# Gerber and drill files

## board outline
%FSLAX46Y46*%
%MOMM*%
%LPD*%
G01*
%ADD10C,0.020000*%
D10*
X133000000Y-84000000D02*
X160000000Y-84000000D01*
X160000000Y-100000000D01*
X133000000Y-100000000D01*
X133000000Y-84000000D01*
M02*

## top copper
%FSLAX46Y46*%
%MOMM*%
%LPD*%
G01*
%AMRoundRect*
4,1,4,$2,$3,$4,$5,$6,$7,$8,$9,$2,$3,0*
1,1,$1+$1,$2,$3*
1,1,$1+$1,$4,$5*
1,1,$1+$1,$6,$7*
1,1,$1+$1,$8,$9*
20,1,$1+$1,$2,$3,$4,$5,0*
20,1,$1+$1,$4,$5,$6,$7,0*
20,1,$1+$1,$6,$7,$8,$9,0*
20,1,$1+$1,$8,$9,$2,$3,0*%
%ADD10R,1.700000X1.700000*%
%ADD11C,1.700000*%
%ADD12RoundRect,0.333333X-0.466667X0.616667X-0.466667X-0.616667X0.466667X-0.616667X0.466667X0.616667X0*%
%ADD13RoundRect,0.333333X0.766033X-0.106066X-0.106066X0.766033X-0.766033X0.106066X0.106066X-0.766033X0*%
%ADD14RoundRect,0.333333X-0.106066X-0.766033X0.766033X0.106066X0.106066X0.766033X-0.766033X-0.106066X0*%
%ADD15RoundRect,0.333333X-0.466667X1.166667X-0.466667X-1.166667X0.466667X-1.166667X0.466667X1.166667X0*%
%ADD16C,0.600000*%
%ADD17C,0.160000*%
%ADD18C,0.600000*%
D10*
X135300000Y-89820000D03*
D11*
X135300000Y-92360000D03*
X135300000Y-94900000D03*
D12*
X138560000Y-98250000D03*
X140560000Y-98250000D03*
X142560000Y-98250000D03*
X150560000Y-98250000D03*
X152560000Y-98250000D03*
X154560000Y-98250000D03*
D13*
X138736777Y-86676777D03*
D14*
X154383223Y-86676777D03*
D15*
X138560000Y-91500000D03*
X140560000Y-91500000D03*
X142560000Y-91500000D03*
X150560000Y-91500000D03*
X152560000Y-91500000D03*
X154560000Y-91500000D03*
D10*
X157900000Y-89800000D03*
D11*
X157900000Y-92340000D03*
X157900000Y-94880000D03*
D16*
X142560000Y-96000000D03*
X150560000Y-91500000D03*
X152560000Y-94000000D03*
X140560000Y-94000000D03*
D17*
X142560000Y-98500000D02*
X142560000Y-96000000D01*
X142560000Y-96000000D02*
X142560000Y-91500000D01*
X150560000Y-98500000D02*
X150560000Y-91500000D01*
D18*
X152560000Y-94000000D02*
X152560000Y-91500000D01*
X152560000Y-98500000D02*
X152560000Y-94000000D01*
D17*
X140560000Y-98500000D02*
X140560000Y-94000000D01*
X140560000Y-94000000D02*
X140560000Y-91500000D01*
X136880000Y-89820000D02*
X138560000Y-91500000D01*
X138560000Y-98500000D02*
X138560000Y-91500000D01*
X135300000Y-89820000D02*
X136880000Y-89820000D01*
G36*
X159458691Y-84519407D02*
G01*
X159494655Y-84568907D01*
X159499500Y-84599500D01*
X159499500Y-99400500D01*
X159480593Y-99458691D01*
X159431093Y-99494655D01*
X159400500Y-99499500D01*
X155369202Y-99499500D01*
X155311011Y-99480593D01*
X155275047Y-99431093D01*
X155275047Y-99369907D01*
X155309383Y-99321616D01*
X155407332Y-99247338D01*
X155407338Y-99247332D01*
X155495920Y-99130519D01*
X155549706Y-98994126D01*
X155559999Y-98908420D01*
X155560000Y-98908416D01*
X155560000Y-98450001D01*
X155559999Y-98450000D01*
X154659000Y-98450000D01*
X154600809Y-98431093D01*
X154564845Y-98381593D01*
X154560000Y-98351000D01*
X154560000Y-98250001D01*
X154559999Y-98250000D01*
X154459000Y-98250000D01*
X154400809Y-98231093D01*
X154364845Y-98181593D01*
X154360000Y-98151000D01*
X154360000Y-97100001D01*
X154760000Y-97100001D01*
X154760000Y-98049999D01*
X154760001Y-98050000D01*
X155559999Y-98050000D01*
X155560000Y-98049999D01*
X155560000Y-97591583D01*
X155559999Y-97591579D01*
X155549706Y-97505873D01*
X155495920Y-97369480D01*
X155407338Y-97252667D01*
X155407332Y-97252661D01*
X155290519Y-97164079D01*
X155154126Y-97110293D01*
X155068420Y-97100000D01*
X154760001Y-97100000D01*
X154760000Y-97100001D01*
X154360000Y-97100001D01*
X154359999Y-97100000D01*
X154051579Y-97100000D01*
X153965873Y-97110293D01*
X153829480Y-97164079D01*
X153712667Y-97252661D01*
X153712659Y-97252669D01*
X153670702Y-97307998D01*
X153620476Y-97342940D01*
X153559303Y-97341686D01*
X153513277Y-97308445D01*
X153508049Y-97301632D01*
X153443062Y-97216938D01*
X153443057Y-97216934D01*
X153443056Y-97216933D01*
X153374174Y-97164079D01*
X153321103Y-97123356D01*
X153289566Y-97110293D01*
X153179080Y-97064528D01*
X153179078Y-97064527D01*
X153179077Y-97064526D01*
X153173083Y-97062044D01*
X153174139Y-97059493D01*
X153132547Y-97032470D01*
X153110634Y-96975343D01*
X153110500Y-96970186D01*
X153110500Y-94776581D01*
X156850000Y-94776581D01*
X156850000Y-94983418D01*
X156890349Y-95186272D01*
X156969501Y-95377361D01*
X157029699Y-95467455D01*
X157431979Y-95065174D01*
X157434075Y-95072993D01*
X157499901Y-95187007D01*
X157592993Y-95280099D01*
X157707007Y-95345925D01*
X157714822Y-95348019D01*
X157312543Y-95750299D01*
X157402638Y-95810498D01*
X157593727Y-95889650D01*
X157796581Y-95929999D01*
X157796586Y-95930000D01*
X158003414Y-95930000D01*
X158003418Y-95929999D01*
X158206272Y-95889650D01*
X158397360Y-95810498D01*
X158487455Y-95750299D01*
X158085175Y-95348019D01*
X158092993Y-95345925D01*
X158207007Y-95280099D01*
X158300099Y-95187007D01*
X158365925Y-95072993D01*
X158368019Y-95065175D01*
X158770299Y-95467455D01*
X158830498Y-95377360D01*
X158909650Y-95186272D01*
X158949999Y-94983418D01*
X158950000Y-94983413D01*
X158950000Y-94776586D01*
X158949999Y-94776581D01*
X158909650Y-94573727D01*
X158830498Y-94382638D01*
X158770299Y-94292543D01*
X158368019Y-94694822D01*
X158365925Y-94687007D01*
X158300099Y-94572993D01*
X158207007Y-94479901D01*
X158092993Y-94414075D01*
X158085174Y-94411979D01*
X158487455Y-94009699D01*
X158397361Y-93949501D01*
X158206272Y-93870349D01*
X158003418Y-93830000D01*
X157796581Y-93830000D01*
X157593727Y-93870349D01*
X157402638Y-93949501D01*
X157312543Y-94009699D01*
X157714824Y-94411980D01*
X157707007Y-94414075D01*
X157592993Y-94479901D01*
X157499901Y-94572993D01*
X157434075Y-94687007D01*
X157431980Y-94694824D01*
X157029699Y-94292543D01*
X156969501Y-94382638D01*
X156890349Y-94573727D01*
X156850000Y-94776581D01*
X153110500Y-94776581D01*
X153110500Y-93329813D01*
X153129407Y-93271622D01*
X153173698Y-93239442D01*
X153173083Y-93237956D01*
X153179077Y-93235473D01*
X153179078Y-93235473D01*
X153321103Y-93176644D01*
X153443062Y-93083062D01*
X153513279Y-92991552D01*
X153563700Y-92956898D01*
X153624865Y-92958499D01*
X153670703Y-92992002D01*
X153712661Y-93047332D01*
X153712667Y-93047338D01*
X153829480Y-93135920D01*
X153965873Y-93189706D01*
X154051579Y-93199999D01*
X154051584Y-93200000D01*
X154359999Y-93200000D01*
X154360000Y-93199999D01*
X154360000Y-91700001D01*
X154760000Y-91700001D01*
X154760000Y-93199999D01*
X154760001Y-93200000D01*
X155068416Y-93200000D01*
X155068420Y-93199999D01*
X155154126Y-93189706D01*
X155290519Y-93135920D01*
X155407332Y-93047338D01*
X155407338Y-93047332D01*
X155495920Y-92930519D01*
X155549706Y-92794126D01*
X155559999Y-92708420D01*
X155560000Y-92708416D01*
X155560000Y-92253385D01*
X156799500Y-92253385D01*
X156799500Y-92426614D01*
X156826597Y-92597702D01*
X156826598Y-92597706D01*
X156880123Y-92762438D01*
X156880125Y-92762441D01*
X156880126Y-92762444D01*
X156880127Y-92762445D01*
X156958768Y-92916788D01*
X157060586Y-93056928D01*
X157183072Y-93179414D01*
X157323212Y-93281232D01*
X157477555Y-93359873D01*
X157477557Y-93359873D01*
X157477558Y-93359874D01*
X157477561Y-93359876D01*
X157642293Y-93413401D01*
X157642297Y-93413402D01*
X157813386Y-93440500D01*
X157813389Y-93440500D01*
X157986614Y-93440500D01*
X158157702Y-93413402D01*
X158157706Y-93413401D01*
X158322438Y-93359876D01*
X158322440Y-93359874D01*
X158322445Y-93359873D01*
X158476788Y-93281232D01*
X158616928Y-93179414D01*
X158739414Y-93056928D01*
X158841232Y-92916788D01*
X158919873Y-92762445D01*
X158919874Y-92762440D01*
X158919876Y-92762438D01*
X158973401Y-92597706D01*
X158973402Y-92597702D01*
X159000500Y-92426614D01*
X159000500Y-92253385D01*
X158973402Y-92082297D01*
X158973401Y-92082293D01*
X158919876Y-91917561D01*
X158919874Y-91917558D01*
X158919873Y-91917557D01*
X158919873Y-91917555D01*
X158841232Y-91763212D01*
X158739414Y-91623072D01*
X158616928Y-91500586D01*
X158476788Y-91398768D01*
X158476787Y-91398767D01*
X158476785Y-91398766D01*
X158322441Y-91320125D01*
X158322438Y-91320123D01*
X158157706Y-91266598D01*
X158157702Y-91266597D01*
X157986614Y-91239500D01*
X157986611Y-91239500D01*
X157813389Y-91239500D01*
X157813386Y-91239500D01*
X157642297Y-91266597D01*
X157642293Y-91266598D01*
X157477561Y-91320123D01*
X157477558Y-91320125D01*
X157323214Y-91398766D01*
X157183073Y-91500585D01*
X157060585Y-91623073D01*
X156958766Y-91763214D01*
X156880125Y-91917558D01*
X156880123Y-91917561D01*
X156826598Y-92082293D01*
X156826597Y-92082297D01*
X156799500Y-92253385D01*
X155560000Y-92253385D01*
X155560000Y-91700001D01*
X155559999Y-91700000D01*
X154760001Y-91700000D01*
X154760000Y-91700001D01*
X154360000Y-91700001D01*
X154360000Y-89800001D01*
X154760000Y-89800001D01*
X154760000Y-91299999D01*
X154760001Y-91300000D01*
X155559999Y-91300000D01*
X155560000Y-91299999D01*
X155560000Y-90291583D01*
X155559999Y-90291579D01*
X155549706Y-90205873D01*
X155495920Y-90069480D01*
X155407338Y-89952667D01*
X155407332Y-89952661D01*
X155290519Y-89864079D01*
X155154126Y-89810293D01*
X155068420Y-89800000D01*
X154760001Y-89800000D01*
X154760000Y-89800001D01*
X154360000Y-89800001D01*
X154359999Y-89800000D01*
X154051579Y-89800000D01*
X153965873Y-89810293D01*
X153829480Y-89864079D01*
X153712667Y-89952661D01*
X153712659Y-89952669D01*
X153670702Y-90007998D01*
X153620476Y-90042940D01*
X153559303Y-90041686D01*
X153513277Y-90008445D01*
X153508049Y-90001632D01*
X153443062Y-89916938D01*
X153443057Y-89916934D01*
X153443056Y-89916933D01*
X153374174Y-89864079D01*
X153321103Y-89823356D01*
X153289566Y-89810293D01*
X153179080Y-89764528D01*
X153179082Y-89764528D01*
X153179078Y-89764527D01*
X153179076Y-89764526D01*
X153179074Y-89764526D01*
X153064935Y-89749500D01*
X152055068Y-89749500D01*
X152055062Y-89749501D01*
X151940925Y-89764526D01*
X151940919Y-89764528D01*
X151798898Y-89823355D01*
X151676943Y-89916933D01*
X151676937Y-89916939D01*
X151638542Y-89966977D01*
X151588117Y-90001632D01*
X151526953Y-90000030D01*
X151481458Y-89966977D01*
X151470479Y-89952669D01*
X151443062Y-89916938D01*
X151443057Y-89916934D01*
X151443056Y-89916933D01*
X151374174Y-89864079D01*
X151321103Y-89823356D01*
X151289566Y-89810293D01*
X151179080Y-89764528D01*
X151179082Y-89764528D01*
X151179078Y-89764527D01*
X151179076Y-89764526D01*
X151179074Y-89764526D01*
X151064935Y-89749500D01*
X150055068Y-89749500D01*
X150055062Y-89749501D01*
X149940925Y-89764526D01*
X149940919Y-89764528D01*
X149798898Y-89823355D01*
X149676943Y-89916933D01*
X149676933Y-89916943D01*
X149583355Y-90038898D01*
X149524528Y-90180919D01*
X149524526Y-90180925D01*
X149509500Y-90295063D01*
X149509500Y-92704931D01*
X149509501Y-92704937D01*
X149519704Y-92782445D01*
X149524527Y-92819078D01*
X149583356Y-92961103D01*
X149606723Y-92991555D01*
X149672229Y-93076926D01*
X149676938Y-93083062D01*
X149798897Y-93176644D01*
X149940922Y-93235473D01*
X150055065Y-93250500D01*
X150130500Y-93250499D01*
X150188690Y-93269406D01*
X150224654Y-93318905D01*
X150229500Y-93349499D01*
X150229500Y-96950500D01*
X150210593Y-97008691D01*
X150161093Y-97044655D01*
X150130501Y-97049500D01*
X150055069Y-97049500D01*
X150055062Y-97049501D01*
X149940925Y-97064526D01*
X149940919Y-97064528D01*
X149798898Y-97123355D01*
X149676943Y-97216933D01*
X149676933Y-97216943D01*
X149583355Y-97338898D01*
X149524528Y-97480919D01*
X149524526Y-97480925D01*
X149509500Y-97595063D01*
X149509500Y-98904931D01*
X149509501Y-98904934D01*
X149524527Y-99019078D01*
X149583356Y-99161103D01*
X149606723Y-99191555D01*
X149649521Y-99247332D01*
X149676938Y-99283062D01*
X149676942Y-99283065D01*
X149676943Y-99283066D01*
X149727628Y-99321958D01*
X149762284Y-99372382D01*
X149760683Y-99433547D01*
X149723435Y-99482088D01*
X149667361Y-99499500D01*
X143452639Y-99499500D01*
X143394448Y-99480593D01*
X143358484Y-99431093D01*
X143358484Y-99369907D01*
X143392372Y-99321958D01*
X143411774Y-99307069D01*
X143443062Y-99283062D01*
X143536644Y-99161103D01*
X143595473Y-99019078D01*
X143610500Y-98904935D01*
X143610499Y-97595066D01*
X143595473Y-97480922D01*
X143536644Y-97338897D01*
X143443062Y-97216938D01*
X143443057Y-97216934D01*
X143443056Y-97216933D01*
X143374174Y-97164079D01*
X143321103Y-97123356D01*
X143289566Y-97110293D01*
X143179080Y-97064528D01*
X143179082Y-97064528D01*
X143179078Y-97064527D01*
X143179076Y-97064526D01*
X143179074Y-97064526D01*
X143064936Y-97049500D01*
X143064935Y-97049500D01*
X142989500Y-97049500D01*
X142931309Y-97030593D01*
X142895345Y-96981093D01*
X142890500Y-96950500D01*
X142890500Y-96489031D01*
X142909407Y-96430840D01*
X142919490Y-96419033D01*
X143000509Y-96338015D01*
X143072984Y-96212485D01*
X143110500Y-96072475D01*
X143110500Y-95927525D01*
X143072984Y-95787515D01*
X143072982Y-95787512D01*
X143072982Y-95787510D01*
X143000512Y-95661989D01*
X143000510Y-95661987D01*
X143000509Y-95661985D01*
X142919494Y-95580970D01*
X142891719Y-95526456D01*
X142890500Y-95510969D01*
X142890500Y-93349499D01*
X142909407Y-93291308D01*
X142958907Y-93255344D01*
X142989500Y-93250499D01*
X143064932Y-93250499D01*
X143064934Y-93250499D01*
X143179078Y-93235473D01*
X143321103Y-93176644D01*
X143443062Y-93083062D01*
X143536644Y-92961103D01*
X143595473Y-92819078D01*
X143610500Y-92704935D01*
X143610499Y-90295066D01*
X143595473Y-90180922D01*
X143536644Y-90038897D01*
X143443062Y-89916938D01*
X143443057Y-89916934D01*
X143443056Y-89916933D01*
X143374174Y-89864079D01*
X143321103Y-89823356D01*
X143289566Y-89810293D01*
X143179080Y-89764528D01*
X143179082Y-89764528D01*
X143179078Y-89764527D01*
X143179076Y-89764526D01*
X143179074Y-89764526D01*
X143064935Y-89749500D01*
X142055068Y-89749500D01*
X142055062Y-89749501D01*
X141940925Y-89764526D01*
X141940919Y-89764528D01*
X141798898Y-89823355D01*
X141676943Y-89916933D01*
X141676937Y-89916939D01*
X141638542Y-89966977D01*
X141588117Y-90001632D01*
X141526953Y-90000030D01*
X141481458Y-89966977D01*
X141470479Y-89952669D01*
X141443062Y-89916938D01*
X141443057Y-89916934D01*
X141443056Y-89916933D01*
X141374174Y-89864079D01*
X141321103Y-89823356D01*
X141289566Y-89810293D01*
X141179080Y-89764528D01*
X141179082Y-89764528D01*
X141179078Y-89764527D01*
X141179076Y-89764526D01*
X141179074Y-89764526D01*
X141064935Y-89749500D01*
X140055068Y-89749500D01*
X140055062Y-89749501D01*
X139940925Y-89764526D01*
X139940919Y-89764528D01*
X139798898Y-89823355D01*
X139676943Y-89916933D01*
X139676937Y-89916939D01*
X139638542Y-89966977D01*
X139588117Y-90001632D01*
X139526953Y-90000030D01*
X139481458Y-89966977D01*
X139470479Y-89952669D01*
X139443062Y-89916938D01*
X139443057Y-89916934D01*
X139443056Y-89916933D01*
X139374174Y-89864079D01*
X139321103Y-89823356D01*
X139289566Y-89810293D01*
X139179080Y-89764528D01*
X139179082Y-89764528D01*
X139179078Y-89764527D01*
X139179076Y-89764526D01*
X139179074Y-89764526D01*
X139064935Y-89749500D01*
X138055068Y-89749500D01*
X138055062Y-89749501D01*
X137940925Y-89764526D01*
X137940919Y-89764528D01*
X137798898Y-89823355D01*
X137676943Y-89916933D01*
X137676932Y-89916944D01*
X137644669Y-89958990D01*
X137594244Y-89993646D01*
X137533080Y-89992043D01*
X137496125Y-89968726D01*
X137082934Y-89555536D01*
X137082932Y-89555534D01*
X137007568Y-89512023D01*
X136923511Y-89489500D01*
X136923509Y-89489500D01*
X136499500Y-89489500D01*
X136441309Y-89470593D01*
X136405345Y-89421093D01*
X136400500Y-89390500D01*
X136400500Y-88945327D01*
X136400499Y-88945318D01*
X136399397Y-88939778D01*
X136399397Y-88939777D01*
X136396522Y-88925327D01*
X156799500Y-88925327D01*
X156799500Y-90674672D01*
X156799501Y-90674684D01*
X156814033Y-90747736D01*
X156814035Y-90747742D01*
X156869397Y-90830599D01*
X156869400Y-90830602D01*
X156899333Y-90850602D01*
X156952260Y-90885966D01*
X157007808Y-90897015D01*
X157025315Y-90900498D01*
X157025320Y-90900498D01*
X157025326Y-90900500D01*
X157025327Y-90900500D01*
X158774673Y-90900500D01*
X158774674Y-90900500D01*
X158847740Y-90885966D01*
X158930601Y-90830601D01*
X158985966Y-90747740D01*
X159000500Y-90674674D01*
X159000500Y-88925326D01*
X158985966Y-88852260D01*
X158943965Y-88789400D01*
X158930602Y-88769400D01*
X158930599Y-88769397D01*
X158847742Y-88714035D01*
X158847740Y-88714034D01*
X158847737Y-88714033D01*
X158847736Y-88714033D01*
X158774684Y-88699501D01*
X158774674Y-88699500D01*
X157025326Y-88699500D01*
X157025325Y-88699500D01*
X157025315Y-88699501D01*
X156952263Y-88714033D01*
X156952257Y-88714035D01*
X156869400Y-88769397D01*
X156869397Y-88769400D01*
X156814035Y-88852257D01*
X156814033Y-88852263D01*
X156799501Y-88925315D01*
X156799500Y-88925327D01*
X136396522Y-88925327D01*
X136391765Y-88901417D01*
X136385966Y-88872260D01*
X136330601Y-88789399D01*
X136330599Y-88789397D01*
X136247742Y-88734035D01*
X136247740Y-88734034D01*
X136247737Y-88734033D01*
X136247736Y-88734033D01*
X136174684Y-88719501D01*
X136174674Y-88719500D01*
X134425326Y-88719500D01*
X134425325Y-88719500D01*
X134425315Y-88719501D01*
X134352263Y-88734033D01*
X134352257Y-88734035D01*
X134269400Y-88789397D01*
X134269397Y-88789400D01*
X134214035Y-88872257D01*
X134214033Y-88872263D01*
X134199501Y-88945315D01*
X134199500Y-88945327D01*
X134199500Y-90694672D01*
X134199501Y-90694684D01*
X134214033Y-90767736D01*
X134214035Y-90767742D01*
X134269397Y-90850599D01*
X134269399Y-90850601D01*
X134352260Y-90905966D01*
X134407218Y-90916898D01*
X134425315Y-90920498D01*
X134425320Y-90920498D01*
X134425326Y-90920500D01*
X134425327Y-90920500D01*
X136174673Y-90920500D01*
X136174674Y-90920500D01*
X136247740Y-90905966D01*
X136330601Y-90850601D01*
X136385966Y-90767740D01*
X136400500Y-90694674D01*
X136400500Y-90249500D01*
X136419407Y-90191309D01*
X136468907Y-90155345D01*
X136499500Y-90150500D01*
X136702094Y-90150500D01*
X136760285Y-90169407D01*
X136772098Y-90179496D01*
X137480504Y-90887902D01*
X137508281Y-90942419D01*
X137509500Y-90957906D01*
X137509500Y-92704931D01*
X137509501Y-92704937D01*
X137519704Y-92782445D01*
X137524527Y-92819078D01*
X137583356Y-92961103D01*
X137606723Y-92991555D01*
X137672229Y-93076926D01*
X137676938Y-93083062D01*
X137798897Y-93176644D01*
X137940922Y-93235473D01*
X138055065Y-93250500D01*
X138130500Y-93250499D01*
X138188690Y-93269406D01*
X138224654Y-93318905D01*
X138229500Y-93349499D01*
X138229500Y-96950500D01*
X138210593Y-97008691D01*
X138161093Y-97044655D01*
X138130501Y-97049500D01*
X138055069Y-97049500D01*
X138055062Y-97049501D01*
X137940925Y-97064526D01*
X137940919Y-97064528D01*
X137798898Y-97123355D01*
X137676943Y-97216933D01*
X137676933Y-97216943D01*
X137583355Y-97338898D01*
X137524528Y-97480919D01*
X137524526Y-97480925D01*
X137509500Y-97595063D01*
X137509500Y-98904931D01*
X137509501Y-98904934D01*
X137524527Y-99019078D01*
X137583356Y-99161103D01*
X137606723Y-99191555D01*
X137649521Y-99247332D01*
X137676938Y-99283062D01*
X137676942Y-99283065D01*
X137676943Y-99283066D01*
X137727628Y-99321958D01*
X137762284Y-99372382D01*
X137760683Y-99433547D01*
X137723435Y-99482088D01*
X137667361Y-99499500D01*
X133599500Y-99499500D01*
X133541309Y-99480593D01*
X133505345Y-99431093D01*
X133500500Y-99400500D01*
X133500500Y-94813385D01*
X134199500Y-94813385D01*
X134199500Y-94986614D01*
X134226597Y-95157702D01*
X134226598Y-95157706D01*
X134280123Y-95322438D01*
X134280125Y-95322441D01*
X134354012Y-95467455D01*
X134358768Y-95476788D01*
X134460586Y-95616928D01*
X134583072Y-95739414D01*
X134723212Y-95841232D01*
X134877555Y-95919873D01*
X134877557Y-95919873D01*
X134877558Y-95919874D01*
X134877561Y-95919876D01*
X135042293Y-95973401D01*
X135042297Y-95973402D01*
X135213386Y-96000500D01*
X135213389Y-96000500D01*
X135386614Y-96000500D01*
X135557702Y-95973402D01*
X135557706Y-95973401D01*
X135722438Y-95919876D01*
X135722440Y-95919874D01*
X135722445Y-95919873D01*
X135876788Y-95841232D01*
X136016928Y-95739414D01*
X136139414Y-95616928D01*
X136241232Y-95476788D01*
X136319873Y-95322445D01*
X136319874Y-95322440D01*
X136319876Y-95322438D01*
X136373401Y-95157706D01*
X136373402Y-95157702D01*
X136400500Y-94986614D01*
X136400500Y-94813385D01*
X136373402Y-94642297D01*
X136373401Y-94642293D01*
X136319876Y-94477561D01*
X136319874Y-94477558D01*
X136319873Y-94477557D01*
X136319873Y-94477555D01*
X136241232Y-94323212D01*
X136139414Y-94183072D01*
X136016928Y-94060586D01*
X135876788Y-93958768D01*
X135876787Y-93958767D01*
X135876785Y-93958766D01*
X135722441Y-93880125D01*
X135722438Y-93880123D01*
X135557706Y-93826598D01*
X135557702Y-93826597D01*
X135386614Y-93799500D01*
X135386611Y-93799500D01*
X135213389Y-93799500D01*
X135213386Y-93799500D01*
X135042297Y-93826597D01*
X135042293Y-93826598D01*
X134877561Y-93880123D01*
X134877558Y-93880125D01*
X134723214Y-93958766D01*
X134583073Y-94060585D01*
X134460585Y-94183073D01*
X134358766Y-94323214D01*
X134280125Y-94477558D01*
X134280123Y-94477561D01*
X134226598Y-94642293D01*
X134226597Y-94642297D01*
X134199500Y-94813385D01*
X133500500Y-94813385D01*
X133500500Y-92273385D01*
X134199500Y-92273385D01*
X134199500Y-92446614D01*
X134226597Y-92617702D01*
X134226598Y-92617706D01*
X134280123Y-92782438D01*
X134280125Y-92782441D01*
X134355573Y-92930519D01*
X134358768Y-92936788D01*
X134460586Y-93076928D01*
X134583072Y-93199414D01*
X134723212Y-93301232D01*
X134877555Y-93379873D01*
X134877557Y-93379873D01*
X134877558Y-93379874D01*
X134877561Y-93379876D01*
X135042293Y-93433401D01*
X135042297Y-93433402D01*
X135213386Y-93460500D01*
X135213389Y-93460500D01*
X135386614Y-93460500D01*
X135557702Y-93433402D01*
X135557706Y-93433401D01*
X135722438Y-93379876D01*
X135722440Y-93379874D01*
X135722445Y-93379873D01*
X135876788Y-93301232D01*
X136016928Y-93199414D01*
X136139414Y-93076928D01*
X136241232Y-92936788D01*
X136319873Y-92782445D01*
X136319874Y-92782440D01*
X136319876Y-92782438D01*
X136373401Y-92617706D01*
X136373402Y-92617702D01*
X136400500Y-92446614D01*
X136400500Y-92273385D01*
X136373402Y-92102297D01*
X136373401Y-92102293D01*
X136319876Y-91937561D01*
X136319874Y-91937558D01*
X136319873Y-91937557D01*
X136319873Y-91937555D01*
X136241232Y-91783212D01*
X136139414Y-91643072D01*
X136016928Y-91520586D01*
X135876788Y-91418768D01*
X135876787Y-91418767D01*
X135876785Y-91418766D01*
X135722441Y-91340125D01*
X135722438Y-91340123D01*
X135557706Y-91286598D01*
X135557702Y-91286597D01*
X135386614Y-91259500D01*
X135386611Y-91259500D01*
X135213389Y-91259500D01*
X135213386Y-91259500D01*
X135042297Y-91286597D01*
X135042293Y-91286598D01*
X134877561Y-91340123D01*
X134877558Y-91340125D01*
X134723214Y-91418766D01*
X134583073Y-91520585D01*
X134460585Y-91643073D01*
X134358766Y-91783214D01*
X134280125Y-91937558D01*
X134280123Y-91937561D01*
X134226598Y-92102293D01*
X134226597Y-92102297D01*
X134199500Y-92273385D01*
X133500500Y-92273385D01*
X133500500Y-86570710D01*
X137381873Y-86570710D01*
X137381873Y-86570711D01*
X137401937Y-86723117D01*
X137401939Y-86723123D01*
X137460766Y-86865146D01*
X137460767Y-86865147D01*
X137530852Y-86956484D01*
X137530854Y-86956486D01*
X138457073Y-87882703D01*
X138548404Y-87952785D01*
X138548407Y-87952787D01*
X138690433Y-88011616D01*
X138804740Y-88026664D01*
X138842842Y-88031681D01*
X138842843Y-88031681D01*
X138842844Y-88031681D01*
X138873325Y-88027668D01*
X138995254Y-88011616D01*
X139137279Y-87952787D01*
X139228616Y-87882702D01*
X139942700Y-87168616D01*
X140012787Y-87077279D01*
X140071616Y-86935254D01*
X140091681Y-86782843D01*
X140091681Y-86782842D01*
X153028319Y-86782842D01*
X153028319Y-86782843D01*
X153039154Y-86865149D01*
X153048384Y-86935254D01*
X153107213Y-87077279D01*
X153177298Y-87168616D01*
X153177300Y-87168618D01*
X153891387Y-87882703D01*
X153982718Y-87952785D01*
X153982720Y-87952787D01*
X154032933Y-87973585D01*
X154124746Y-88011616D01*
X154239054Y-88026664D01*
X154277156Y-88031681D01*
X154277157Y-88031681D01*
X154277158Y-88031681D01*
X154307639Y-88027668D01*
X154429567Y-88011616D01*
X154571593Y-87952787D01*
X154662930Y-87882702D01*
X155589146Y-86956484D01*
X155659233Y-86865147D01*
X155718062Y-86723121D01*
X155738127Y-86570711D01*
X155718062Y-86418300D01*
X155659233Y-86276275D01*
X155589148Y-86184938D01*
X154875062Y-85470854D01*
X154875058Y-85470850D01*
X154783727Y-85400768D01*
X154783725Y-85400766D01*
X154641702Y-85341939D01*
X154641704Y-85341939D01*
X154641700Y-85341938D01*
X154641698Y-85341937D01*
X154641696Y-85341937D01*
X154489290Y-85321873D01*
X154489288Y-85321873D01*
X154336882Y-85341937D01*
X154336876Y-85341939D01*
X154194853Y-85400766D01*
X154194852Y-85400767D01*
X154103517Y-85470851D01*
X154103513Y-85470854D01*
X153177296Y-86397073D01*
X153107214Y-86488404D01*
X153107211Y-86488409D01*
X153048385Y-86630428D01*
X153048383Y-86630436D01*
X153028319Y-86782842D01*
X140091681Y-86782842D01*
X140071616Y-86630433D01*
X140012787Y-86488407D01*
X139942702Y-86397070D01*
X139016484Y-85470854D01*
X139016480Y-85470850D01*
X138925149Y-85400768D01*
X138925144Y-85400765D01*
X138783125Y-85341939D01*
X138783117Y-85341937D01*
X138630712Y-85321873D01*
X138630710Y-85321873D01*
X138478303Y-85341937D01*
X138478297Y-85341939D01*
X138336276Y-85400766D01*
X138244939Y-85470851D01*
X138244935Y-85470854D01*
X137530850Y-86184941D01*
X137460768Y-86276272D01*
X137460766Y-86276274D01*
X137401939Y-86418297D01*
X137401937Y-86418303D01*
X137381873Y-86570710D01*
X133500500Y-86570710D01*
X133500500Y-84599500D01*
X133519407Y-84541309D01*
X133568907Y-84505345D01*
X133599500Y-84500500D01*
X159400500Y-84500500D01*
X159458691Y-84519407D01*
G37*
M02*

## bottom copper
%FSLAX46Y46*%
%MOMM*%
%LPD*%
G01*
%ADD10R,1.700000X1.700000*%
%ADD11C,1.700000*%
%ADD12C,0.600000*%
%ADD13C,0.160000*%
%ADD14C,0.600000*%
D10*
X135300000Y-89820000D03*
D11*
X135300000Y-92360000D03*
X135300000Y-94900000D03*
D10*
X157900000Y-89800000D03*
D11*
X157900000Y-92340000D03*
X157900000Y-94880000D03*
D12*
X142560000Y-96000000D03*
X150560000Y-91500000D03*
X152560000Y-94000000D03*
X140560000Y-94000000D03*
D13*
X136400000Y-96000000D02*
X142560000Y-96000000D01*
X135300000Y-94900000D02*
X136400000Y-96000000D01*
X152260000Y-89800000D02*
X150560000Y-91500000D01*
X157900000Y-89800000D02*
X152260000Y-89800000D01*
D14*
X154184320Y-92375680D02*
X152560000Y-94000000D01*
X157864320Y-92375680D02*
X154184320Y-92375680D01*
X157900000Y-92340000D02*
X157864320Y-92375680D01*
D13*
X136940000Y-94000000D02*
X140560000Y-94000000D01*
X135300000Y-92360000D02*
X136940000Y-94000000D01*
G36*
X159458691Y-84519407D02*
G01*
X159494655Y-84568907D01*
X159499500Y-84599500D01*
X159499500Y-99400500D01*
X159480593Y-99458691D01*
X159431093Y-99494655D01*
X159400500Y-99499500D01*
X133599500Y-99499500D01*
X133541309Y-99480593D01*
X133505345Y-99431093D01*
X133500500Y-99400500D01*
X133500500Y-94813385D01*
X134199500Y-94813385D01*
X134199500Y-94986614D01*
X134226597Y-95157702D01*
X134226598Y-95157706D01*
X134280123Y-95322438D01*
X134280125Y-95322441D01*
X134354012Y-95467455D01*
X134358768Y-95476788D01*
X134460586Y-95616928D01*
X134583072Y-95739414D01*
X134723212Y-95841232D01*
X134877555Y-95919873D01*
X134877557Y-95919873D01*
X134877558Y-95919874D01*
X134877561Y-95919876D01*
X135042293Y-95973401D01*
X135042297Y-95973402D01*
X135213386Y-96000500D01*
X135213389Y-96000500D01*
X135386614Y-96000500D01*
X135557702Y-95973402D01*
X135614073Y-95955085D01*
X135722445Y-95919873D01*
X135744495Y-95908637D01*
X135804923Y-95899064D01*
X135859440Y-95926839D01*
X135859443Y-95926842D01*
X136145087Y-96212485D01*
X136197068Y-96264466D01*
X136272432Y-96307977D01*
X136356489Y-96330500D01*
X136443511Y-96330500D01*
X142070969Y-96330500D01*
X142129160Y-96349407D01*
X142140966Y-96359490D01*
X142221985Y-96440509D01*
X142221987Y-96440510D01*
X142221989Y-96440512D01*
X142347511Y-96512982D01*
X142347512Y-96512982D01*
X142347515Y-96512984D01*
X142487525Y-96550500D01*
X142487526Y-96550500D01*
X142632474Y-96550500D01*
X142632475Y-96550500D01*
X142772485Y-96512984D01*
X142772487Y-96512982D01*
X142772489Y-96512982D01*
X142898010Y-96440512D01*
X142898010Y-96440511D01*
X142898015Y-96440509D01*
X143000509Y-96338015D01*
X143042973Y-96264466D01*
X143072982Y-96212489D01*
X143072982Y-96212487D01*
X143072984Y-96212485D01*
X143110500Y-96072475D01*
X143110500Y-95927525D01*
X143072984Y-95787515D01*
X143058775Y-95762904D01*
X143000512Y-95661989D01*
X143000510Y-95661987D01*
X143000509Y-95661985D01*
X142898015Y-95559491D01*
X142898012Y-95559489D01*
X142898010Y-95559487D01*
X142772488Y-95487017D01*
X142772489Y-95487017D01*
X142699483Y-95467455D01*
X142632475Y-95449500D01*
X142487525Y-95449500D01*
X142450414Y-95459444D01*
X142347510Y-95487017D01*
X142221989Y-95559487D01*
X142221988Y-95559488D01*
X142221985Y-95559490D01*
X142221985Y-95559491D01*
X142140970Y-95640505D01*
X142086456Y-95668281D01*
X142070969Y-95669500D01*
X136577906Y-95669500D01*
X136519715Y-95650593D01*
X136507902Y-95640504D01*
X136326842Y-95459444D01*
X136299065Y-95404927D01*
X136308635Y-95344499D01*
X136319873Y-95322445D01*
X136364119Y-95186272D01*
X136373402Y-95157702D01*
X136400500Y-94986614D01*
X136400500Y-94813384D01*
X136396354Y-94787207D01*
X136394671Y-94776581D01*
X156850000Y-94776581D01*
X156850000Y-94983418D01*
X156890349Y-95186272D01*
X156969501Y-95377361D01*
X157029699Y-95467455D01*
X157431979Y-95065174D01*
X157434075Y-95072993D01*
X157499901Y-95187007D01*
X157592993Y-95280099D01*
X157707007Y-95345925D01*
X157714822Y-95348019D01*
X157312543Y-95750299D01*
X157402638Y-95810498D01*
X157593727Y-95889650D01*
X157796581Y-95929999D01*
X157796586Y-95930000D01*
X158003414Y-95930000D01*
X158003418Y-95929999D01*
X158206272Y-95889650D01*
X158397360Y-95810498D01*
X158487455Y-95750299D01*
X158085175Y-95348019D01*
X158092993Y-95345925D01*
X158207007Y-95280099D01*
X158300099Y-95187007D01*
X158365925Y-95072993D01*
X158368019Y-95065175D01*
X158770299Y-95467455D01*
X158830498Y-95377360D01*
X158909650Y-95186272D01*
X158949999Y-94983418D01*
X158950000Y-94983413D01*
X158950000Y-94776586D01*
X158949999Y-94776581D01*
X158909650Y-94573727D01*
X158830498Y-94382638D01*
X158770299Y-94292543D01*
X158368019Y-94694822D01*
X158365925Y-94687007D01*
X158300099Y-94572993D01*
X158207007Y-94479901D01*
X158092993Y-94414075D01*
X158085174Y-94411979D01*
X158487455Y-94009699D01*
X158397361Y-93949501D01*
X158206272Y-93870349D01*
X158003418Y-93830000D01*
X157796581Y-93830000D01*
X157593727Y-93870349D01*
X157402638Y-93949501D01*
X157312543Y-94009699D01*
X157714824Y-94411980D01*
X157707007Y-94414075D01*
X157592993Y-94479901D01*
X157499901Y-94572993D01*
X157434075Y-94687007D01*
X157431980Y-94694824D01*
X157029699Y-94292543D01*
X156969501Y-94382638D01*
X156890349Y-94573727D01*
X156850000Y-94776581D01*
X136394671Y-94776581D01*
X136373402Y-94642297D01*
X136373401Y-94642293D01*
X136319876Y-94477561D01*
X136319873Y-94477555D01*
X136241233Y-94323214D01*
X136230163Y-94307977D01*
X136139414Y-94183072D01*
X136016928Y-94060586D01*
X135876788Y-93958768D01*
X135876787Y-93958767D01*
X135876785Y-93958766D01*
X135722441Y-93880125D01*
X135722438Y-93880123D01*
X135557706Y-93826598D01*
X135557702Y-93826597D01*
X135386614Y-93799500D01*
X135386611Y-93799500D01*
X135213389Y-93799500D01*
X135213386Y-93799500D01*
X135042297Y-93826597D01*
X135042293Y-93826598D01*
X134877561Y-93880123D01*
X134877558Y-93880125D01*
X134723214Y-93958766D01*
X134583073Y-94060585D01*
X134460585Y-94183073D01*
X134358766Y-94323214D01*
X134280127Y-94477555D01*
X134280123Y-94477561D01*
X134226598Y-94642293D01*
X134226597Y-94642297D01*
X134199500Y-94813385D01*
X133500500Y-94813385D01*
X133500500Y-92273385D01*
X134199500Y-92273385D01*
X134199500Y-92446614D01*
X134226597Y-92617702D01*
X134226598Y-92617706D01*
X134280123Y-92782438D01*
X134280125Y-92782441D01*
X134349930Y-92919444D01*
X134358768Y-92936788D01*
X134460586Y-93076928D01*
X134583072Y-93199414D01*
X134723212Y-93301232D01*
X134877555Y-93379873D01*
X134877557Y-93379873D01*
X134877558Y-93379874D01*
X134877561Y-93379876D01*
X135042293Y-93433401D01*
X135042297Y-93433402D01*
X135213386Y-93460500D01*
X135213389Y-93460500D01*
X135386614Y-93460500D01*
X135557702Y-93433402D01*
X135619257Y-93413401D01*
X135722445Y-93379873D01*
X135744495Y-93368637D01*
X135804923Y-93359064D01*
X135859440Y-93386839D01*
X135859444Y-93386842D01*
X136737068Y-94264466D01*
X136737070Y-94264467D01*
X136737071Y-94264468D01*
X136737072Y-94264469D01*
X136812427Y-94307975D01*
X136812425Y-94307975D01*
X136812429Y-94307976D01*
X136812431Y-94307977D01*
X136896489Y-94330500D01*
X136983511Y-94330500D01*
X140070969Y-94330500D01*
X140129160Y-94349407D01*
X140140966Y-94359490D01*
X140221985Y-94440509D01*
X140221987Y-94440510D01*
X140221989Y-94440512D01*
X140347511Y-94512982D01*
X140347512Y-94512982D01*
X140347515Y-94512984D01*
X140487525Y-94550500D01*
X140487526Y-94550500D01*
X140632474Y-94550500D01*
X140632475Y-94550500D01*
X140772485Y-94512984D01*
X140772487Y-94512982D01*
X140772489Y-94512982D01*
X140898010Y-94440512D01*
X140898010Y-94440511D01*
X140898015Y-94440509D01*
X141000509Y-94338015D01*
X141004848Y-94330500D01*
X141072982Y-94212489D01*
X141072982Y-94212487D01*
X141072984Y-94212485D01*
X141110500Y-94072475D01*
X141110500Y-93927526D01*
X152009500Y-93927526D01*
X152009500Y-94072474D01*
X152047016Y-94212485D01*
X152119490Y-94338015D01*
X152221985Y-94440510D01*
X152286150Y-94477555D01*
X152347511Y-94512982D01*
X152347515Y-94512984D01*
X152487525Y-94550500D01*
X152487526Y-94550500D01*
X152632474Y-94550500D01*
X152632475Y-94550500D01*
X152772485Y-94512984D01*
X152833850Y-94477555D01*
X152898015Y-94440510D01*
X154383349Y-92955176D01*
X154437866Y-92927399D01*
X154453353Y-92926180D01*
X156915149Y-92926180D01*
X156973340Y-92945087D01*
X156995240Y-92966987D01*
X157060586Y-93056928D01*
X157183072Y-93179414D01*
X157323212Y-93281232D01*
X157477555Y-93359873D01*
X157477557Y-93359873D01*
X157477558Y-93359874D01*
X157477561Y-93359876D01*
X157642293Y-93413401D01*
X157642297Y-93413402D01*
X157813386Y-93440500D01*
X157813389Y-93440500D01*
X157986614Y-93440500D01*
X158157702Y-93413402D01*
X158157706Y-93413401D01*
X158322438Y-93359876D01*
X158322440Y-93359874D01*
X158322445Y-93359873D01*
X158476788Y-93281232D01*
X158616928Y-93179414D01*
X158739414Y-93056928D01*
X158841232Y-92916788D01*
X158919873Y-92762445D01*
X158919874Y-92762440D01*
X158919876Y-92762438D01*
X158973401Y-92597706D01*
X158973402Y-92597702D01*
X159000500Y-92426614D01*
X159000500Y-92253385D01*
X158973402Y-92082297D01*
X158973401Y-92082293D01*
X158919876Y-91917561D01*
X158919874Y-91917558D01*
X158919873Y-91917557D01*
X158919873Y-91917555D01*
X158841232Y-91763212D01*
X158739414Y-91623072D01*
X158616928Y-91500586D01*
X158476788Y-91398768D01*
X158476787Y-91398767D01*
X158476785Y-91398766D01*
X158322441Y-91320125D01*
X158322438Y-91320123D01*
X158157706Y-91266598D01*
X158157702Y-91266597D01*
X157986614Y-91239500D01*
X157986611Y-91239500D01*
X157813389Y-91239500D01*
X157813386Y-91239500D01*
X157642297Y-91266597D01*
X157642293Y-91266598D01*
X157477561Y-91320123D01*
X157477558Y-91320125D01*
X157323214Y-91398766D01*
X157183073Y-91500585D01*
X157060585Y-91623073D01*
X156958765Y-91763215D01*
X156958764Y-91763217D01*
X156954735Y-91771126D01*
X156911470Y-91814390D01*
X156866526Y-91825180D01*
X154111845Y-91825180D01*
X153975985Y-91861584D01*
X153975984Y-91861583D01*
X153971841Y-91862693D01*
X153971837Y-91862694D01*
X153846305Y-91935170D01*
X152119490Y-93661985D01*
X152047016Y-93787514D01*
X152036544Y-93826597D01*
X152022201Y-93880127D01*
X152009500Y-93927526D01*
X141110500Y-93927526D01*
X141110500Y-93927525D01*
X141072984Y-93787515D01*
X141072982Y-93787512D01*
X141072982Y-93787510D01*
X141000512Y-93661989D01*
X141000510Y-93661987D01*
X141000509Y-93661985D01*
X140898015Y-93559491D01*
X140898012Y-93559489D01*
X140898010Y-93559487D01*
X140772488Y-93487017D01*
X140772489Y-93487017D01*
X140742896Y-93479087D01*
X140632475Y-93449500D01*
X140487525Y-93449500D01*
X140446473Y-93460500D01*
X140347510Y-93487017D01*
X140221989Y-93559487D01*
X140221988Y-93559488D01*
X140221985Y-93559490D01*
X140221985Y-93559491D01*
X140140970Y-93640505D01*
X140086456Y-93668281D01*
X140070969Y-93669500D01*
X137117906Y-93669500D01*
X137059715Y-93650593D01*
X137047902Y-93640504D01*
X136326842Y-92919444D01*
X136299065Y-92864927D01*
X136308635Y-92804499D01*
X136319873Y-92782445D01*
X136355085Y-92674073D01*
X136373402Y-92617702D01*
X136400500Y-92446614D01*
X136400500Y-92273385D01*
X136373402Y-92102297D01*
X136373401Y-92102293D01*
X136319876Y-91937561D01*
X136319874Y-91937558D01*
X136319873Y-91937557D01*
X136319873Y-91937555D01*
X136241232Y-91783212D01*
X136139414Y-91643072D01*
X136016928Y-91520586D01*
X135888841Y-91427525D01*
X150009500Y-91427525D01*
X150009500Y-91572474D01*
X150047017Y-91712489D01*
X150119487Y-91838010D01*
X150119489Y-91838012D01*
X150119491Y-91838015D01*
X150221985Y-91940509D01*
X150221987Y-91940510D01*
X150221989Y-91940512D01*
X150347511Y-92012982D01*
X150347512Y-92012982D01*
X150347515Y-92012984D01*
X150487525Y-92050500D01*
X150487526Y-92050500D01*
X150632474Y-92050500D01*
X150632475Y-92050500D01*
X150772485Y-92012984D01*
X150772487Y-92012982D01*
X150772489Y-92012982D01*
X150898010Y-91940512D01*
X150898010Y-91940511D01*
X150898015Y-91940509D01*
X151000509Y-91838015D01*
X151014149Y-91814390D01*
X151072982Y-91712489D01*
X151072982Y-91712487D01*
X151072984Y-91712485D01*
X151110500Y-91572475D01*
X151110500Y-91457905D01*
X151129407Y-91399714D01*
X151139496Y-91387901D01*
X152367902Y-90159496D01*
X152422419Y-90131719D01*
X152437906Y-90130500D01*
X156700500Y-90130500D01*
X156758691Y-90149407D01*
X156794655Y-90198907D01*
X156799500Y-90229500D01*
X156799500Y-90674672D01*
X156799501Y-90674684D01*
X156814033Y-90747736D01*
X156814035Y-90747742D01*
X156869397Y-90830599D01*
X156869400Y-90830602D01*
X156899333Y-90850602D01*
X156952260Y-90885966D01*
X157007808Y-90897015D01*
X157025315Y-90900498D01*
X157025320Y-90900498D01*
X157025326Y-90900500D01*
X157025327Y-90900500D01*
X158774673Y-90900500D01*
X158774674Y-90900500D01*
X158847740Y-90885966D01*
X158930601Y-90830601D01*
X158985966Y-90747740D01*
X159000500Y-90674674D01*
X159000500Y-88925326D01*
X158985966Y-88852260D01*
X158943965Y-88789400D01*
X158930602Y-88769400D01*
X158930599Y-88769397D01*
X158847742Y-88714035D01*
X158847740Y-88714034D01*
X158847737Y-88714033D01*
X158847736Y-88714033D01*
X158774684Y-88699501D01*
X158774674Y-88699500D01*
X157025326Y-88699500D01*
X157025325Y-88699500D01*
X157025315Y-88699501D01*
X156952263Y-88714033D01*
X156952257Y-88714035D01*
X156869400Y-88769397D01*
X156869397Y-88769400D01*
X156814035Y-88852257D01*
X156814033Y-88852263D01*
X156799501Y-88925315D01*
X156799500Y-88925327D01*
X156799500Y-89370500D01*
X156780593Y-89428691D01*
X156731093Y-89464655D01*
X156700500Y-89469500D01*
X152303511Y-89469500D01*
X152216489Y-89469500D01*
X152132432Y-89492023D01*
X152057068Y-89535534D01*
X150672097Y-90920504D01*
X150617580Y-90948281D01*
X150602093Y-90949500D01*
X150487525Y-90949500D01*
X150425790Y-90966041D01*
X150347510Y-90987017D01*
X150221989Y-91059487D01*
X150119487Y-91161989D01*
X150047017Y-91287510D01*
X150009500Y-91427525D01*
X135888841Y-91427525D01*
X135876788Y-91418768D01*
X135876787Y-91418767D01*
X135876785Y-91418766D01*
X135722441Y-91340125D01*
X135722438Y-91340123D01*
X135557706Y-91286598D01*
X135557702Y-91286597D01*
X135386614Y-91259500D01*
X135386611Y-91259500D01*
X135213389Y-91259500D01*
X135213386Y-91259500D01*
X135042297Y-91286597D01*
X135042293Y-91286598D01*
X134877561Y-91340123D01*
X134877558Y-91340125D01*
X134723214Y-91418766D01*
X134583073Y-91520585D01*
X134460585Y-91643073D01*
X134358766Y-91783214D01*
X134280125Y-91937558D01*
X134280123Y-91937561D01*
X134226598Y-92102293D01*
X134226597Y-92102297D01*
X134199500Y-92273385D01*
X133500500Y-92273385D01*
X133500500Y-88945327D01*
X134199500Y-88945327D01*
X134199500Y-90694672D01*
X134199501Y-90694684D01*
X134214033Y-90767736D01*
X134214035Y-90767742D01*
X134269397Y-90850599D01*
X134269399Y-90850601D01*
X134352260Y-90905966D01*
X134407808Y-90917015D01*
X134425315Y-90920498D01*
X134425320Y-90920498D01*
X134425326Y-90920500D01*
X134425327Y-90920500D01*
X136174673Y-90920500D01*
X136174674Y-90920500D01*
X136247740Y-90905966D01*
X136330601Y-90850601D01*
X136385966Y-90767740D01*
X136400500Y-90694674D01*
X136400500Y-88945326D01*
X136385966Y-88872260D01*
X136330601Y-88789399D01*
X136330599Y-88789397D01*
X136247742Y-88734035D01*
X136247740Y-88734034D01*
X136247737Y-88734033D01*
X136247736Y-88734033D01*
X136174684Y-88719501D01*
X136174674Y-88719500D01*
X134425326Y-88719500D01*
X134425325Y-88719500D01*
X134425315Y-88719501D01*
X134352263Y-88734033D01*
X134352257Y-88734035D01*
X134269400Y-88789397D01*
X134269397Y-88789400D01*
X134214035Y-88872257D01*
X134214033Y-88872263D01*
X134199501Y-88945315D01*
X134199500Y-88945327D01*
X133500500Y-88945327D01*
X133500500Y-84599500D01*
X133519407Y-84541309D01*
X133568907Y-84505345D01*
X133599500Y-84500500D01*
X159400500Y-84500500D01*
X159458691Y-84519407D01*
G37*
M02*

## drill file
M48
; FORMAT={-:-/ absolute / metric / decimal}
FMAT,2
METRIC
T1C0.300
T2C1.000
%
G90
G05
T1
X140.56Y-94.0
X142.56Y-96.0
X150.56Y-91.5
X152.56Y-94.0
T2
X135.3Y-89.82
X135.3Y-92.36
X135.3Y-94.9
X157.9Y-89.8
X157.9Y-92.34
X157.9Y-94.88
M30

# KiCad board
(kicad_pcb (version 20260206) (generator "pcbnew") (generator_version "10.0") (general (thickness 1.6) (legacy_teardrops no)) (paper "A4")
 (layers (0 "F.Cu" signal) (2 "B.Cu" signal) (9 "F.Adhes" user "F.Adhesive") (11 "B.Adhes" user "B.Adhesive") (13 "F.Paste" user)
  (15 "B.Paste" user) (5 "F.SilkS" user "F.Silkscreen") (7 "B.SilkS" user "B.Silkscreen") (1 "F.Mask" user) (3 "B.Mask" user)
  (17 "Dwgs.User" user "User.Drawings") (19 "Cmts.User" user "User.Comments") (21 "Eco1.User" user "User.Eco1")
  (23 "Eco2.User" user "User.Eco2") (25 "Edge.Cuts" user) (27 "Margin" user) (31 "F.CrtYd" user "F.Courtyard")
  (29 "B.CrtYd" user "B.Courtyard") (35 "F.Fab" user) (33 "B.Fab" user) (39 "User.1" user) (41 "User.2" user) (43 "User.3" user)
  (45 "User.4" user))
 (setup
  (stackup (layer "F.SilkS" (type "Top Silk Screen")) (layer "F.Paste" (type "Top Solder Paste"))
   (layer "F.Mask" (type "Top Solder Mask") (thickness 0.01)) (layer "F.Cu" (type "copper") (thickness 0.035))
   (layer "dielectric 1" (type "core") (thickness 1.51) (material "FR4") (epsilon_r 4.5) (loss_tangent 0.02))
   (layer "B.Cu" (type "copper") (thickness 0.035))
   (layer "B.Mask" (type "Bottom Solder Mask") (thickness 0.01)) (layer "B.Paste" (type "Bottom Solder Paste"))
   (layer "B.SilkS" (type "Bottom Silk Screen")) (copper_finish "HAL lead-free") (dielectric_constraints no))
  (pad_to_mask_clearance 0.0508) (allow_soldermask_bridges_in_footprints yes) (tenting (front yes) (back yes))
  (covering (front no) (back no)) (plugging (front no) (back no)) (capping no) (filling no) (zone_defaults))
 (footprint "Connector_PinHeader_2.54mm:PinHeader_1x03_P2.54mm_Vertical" (layer "F.Cu") (at 135.3 89.82)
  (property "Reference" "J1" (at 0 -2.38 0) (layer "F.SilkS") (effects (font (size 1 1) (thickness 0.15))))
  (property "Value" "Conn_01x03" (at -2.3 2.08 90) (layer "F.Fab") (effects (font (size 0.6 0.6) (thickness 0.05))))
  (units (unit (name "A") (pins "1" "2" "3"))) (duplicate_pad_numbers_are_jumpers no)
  (pad "1" thru_hole rect (at 0 0) (size 1.7 1.7) (drill 1) (layers "*.Cu" "*.Mask") (remove_unused_layers no) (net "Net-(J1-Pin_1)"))
  (pad "2" thru_hole circle (at 0 2.54) (size 1.7 1.7) (drill 1) (layers "*.Cu" "*.Mask") (remove_unused_layers no) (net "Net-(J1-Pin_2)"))
  (pad "3" thru_hole circle (at 0 5.08) (size 1.7 1.7) (drill 1) (layers "*.Cu" "*.Mask") (remove_unused_layers no) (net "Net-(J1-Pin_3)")))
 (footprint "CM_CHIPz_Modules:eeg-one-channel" (layer "F.Cu") (at 146.56 91.5)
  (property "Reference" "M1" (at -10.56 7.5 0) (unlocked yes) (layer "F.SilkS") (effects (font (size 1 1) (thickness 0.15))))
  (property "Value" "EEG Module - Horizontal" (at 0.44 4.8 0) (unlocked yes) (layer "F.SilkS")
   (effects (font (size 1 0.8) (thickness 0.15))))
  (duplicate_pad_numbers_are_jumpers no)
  (pad "1" smd roundrect (at -8 7 270) (size 1.9 1.6) (drill (offset -0.25 0)) (layers "F.Cu" "F.Mask" "F.Paste")
   (roundrect_rratio 0.2083333333) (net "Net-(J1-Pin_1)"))
  (pad "2" smd roundrect (at -6 7 270) (size 1.9 1.6) (drill (offset -0.25 0)) (layers "F.Cu" "F.Mask" "F.Paste")
   (roundrect_rratio 0.2083333333) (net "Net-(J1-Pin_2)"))
  (pad "3" smd roundrect (at -4 7 270) (size 1.9 1.6) (drill (offset -0.25 0)) (layers "F.Cu" "F.Mask" "F.Paste")
   (roundrect_rratio 0.2083333333) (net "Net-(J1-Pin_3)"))
  (pad "4" smd roundrect (at 4 7 270) (size 1.9 1.6) (drill (offset -0.25 0)) (layers "F.Cu" "F.Mask" "F.Paste")
   (roundrect_rratio 0.2083333333) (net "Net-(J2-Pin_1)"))
  (pad "5" smd roundrect (at 6 7 270) (size 1.9 1.6) (drill (offset -0.25 0)) (layers "F.Cu" "F.Mask" "F.Paste")
   (roundrect_rratio 0.2083333333) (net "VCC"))
  (pad "6" smd roundrect (at 8 7 270) (size 1.9 1.6) (drill (offset -0.25 0)) (layers "F.Cu" "F.Mask" "F.Paste")
   (roundrect_rratio 0.2083333333) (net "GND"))
  (pad "7" smd roundrect (at -8 -5 135) (size 1.9 1.6) (drill (offset -0.25 0)) (layers "F.Cu" "F.Mask" "F.Paste")
   (roundrect_rratio 0.2083333333))
  (pad "8" smd roundrect (at 8 -5 45) (size 1.9 1.6) (drill (offset -0.25 0)) (layers "F.Cu" "F.Mask" "F.Paste")
   (roundrect_rratio 0.2083333333))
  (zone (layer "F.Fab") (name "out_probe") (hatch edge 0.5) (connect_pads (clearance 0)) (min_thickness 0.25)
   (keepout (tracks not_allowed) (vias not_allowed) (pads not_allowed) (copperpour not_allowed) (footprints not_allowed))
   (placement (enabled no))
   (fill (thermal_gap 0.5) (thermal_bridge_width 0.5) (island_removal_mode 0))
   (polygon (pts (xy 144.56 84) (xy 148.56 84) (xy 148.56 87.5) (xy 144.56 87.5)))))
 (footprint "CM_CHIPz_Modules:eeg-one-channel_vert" (layer "F.Cu") (at 146.56 91.5)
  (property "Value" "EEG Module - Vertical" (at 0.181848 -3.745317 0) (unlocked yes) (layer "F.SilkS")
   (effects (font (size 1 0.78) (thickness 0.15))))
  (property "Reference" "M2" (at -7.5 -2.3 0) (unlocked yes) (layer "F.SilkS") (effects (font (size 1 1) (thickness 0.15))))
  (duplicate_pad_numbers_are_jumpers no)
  (pad "1" smd roundrect (at -8 0 270) (size 3 1.6) (layers "F.Cu" "F.Mask" "F.Paste") (roundrect_rratio 0.2083333333)
   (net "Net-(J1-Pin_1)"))
  (pad "2" smd roundrect (at -6 0 270) (size 3 1.6) (layers "F.Cu" "F.Mask" "F.Paste") (roundrect_rratio 0.2083333333)
   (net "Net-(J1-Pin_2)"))
  (pad "3" smd roundrect (at -4 0 270) (size 3 1.6) (layers "F.Cu" "F.Mask" "F.Paste") (roundrect_rratio 0.2083333333)
   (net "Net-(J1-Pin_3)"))
  (pad "4" smd roundrect (at 4 0 270) (size 3 1.6) (layers "F.Cu" "F.Mask" "F.Paste") (roundrect_rratio 0.2083333333) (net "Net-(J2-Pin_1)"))
  (pad "5" smd roundrect (at 6 0 270) (size 3 1.6) (layers "F.Cu" "F.Mask" "F.Paste") (roundrect_rratio 0.2083333333) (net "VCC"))
  (pad "6" smd roundrect (at 8 0 270) (size 3 1.6) (layers "F.Cu" "F.Mask" "F.Paste") (roundrect_rratio 0.2083333333) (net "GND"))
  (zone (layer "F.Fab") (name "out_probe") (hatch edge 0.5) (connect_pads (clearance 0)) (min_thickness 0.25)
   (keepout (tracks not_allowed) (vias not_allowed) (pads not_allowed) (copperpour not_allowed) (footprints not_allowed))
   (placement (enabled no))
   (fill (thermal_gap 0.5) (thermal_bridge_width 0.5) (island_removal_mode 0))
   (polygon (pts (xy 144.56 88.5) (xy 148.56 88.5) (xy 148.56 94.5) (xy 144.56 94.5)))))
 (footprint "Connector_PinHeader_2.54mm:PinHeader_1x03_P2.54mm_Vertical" (layer "F.Cu") (at 157.9 89.8)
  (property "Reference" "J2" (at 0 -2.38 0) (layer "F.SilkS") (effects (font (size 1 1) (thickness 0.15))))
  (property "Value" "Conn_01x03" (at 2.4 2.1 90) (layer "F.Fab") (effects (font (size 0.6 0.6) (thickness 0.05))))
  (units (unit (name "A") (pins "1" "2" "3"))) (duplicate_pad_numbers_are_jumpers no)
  (pad "1" thru_hole rect (at 0 0) (size 1.7 1.7) (drill 1) (layers "*.Cu" "*.Mask") (remove_unused_layers no) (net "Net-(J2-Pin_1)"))
  (pad "2" thru_hole circle (at 0 2.54) (size 1.7 1.7) (drill 1) (layers "*.Cu" "*.Mask") (remove_unused_layers no) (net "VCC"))
  (pad "3" thru_hole circle (at 0 5.08) (size 1.7 1.7) (drill 1) (layers "*.Cu" "*.Mask") (remove_unused_layers no) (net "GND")))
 (gr_poly (pts (xy 133 84) (xy 160 84) (xy 160 100) (xy 133 100)) (stroke (width 0.02) (type solid)) (fill no) (layer "Edge.Cuts"))
 (segment (start 142.56 98.5) (end 142.56 96) (width 0.16) (layer "F.Cu") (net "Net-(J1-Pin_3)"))
 (segment (start 142.56 96) (end 142.56 91.5) (width 0.16) (layer "F.Cu") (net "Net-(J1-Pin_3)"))
 (via (at 142.56 96) (size 0.6) (drill 0.3) (layers "F.Cu" "B.Cu") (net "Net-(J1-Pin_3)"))
 (segment (start 136.4 96) (end 142.56 96) (width 0.16) (layer "B.Cu") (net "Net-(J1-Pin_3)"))
 (segment (start 135.3 94.9) (end 136.4 96) (width 0.16) (layer "B.Cu") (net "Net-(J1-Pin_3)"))
 (segment (start 150.56 98.5) (end 150.56 91.5) (width 0.16) (layer "F.Cu") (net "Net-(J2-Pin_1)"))
 (via (at 150.56 91.5) (size 0.6) (drill 0.3) (layers "F.Cu" "B.Cu") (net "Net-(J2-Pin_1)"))
 (segment (start 152.26 89.8) (end 150.56 91.5) (width 0.16) (layer "B.Cu") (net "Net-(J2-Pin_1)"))
 (segment (start 157.9 89.8) (end 152.26 89.8) (width 0.16) (layer "B.Cu") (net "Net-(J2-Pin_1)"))
 (segment (start 152.56 94) (end 152.56 91.5) (width 0.6) (layer "F.Cu") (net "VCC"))
 (segment (start 152.56 98.5) (end 152.56 94) (width 0.6) (layer "F.Cu") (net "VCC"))
 (via (at 152.56 94) (size 0.6) (drill 0.3) (layers "F.Cu" "B.Cu") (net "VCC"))
 (segment (start 154.18432 92.37568) (end 152.56 94) (width 0.6) (layer "B.Cu") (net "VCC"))
 (segment (start 157.86432 92.37568) (end 154.18432 92.37568) (width 0.6) (layer "B.Cu") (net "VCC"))
 (segment (start 157.9 92.34) (end 157.86432 92.37568) (width 0.6) (layer "B.Cu") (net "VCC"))
 (segment (start 140.56 98.5) (end 140.56 94) (width 0.16) (layer "F.Cu") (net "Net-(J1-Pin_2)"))
 (segment (start 140.56 94) (end 140.56 91.5) (width 0.16) (layer "F.Cu") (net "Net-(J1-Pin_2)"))
 (via (at 140.56 94) (size 0.6) (drill 0.3) (layers "F.Cu" "B.Cu") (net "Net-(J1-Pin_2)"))
 (segment (start 136.94 94) (end 140.56 94) (width 0.16) (layer "B.Cu") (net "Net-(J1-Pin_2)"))
 (segment (start 135.3 92.36) (end 136.94 94) (width 0.16) (layer "B.Cu") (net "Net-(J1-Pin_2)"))
 (segment (start 136.88 89.82) (end 138.56 91.5) (width 0.16) (layer "F.Cu") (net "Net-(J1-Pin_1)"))
 (segment (start 138.56 98.5) (end 138.56 91.5) (width 0.16) (layer "F.Cu") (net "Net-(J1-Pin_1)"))
 (segment (start 135.3 89.82) (end 136.88 89.82) (width 0.16) (layer "F.Cu") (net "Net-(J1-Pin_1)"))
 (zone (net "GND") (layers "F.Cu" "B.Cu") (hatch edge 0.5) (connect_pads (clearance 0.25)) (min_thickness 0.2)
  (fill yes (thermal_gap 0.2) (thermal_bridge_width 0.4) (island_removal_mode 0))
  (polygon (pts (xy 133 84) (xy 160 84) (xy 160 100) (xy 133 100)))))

